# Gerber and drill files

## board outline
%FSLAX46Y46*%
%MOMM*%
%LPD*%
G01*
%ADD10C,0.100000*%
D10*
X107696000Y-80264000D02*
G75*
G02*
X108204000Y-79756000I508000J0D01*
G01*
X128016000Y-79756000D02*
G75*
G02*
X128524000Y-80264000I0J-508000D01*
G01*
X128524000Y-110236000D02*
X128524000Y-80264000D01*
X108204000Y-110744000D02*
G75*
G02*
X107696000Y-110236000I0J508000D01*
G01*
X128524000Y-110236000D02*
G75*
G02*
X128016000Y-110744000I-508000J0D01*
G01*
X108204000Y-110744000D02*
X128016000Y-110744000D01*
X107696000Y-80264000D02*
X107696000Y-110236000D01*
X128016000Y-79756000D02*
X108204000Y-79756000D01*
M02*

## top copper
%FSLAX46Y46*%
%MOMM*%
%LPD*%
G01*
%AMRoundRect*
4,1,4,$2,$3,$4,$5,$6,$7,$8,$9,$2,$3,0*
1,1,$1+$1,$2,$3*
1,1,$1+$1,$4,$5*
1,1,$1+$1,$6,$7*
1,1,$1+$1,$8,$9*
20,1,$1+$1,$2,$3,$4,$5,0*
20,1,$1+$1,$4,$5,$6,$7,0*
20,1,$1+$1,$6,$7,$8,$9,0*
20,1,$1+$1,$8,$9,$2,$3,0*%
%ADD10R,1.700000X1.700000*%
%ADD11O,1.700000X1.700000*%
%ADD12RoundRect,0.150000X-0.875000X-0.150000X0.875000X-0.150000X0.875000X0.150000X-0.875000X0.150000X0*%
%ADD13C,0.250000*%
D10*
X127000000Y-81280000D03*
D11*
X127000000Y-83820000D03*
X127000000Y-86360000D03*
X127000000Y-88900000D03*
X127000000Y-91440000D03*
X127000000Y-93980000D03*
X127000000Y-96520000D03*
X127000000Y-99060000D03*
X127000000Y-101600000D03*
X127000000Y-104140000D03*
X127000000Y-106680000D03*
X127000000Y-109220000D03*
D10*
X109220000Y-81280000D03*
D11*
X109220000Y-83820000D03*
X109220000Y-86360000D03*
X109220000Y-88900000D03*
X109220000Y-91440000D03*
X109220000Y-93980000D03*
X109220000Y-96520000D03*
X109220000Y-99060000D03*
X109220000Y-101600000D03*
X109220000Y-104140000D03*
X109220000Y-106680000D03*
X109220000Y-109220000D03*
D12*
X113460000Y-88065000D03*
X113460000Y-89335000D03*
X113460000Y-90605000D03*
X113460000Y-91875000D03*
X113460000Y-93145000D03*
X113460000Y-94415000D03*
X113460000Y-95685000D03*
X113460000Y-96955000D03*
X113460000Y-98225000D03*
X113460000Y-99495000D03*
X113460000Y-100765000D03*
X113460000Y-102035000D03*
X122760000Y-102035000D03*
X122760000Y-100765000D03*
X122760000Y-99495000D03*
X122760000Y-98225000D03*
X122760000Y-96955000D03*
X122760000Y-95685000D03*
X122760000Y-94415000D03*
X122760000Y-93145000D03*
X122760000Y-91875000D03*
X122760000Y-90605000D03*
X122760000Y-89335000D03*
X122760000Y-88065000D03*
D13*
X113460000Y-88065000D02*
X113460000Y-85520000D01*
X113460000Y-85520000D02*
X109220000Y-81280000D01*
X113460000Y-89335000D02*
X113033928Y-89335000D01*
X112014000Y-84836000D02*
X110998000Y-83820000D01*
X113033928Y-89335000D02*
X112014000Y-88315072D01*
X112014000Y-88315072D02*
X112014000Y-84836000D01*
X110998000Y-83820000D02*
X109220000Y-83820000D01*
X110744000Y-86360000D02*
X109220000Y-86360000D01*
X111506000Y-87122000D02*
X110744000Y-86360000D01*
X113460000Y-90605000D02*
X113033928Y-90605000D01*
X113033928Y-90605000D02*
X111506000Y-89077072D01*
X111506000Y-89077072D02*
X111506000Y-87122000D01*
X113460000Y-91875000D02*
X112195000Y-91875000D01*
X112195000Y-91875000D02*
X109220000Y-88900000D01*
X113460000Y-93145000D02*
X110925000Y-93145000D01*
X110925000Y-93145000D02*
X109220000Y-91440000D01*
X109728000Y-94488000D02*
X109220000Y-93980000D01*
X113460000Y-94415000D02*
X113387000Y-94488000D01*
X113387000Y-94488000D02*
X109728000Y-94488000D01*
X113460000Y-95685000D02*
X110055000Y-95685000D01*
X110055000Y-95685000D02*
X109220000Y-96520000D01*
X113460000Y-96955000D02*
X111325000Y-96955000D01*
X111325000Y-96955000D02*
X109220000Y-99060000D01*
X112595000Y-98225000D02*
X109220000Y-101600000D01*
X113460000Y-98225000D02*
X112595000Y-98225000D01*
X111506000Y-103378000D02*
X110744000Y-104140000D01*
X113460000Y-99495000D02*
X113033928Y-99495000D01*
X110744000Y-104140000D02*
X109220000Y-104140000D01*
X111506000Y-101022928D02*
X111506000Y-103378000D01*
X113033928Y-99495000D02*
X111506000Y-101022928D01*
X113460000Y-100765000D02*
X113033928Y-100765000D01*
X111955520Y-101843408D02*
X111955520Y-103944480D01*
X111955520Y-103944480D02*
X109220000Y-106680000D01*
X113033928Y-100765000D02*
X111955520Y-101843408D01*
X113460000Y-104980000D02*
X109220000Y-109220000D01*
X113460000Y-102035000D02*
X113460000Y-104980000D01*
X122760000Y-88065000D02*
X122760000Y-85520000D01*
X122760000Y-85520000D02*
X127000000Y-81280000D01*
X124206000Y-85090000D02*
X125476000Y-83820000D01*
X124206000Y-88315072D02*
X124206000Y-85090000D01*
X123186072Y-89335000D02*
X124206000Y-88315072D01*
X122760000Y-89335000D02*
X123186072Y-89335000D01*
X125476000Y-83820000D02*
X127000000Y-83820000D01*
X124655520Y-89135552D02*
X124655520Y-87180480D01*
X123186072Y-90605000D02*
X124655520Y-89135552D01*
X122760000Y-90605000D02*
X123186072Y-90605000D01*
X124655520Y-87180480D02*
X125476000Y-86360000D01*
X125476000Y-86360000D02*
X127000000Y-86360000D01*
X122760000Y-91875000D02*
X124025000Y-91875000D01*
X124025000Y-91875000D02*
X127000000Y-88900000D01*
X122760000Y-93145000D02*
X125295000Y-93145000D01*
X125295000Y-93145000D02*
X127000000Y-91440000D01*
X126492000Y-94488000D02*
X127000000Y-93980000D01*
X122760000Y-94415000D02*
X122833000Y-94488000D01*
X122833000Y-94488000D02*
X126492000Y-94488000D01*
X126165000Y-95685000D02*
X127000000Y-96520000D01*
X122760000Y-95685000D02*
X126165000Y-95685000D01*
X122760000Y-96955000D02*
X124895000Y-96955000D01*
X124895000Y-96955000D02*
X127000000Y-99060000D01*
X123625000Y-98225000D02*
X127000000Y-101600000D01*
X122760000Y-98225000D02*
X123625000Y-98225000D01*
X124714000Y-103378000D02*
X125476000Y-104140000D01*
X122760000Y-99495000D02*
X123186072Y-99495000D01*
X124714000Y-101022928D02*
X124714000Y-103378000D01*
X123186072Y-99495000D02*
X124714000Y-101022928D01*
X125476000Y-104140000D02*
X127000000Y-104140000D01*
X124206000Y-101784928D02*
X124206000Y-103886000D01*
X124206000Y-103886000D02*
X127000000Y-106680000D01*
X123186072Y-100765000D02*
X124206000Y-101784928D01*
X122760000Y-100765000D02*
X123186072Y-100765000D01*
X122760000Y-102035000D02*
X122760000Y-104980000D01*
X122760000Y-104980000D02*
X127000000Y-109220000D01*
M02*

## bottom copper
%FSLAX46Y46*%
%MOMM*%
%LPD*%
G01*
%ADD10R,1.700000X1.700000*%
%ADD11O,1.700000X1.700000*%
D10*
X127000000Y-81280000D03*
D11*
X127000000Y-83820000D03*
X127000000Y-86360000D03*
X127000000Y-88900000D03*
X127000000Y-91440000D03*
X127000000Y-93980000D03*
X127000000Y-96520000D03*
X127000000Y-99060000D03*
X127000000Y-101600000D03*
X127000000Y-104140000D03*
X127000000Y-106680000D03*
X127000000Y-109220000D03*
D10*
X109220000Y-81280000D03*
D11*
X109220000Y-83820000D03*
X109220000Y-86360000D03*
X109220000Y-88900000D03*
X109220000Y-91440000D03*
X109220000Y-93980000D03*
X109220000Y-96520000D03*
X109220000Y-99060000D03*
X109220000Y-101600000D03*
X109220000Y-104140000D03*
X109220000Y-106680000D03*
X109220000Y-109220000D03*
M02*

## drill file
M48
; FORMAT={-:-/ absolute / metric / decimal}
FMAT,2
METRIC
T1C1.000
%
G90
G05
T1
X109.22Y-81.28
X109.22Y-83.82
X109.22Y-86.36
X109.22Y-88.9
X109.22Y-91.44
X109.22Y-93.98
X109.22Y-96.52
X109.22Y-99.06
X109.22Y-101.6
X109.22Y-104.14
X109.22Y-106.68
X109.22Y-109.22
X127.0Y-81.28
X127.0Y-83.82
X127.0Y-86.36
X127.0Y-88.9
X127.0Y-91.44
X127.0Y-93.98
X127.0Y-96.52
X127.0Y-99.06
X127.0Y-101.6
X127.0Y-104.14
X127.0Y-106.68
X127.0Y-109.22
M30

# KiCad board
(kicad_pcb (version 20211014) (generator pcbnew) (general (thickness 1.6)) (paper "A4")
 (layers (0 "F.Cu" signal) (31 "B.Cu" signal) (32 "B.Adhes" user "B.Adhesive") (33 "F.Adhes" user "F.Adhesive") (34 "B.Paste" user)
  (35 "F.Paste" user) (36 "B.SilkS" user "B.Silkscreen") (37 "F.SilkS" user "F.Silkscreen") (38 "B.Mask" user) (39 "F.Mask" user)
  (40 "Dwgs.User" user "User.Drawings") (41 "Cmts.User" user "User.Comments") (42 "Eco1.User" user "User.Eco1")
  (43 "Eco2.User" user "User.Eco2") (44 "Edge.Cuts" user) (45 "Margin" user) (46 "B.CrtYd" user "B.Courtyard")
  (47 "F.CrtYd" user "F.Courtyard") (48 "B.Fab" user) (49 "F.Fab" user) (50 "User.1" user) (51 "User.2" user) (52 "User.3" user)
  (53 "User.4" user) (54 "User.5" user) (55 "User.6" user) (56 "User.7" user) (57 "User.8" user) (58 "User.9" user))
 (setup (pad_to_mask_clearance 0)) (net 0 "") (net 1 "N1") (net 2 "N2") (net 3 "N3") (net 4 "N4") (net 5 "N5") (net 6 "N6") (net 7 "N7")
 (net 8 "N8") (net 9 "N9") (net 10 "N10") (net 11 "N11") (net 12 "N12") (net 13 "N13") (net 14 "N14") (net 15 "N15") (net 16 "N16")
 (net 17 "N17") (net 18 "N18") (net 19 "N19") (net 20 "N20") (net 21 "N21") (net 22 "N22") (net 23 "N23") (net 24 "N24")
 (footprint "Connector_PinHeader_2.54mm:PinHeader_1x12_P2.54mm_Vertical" (layer "F.Cu") (at 127 81.28)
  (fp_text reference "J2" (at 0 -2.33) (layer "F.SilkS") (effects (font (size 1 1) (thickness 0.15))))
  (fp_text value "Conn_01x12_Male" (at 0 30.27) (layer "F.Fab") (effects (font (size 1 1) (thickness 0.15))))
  (pad "1" thru_hole rect locked (at 0 0) (size 1.7 1.7) (drill 1) (layers *.Cu *.Mask) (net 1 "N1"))
  (pad "2" thru_hole oval locked (at 0 2.54) (size 1.7 1.7) (drill 1) (layers *.Cu *.Mask) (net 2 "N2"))
  (pad "3" thru_hole oval locked (at 0 5.08) (size 1.7 1.7) (drill 1) (layers *.Cu *.Mask) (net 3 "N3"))
  (pad "4" thru_hole oval locked (at 0 7.62) (size 1.7 1.7) (drill 1) (layers *.Cu *.Mask) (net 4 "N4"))
  (pad "5" thru_hole oval locked (at 0 10.16) (size 1.7 1.7) (drill 1) (layers *.Cu *.Mask) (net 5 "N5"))
  (pad "6" thru_hole oval locked (at 0 12.7) (size 1.7 1.7) (drill 1) (layers *.Cu *.Mask) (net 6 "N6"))
  (pad "7" thru_hole oval locked (at 0 15.24) (size 1.7 1.7) (drill 1) (layers *.Cu *.Mask) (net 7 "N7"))
  (pad "8" thru_hole oval locked (at 0 17.78) (size 1.7 1.7) (drill 1) (layers *.Cu *.Mask) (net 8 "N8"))
  (pad "9" thru_hole oval locked (at 0 20.32) (size 1.7 1.7) (drill 1) (layers *.Cu *.Mask) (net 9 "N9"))
  (pad "10" thru_hole oval locked (at 0 22.86) (size 1.7 1.7) (drill 1) (layers *.Cu *.Mask) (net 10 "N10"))
  (pad "11" thru_hole oval locked (at 0 25.4) (size 1.7 1.7) (drill 1) (layers *.Cu *.Mask) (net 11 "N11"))
  (pad "12" thru_hole oval locked (at 0 27.94) (size 1.7 1.7) (drill 1) (layers *.Cu *.Mask) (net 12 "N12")))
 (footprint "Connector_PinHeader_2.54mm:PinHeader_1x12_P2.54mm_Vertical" (layer "F.Cu") (at 109.22 81.28)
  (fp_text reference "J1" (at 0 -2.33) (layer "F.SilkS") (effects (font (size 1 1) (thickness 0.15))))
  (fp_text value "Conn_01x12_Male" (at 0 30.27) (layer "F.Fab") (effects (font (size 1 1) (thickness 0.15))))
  (pad "1" thru_hole rect locked (at 0 0) (size 1.7 1.7) (drill 1) (layers *.Cu *.Mask) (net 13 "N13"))
  (pad "2" thru_hole oval locked (at 0 2.54) (size 1.7 1.7) (drill 1) (layers *.Cu *.Mask) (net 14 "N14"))
  (pad "3" thru_hole oval locked (at 0 5.08) (size 1.7 1.7) (drill 1) (layers *.Cu *.Mask) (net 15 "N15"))
  (pad "4" thru_hole oval locked (at 0 7.62) (size 1.7 1.7) (drill 1) (layers *.Cu *.Mask) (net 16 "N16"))
  (pad "5" thru_hole oval locked (at 0 10.16) (size 1.7 1.7) (drill 1) (layers *.Cu *.Mask) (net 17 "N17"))
  (pad "6" thru_hole oval locked (at 0 12.7) (size 1.7 1.7) (drill 1) (layers *.Cu *.Mask) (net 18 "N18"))
  (pad "7" thru_hole oval locked (at 0 15.24) (size 1.7 1.7) (drill 1) (layers *.Cu *.Mask) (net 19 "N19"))
  (pad "8" thru_hole oval locked (at 0 17.78) (size 1.7 1.7) (drill 1) (layers *.Cu *.Mask) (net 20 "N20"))
  (pad "9" thru_hole oval locked (at 0 20.32) (size 1.7 1.7) (drill 1) (layers *.Cu *.Mask) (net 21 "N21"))
  (pad "10" thru_hole oval locked (at 0 22.86) (size 1.7 1.7) (drill 1) (layers *.Cu *.Mask) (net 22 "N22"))
  (pad "11" thru_hole oval locked (at 0 25.4) (size 1.7 1.7) (drill 1) (layers *.Cu *.Mask) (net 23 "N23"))
  (pad "12" thru_hole oval locked (at 0 27.94) (size 1.7 1.7) (drill 1) (layers *.Cu *.Mask) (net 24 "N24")))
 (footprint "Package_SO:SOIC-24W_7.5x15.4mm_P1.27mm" (layer "F.Cu") (at 118.11 95.05)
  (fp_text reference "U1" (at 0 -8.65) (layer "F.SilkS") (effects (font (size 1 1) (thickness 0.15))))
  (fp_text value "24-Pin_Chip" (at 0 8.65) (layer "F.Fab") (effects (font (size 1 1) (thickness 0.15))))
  (pad "1" smd roundrect locked (at -4.65 -6.985) (size 2.05 0.6) (layers "F.Cu" "F.Paste" "F.Mask") (roundrect_rratio 0.25) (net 13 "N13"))
  (pad "2" smd roundrect locked (at -4.65 -5.715) (size 2.05 0.6) (layers "F.Cu" "F.Paste" "F.Mask") (roundrect_rratio 0.25) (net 14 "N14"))
  (pad "3" smd roundrect locked (at -4.65 -4.445) (size 2.05 0.6) (layers "F.Cu" "F.Paste" "F.Mask") (roundrect_rratio 0.25) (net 15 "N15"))
  (pad "4" smd roundrect locked (at -4.65 -3.175) (size 2.05 0.6) (layers "F.Cu" "F.Paste" "F.Mask") (roundrect_rratio 0.25) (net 16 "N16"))
  (pad "5" smd roundrect locked (at -4.65 -1.905) (size 2.05 0.6) (layers "F.Cu" "F.Paste" "F.Mask") (roundrect_rratio 0.25) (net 17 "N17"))
  (pad "6" smd roundrect locked (at -4.65 -0.635) (size 2.05 0.6) (layers "F.Cu" "F.Paste" "F.Mask") (roundrect_rratio 0.25) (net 18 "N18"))
  (pad "7" smd roundrect locked (at -4.65 0.635) (size 2.05 0.6) (layers "F.Cu" "F.Paste" "F.Mask") (roundrect_rratio 0.25) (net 19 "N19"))
  (pad "8" smd roundrect locked (at -4.65 1.905) (size 2.05 0.6) (layers "F.Cu" "F.Paste" "F.Mask") (roundrect_rratio 0.25) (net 20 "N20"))
  (pad "9" smd roundrect locked (at -4.65 3.175) (size 2.05 0.6) (layers "F.Cu" "F.Paste" "F.Mask") (roundrect_rratio 0.25) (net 21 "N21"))
  (pad "10" smd roundrect locked (at -4.65 4.445) (size 2.05 0.6) (layers "F.Cu" "F.Paste" "F.Mask") (roundrect_rratio 0.25) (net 22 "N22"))
  (pad "11" smd roundrect locked (at -4.65 5.715) (size 2.05 0.6) (layers "F.Cu" "F.Paste" "F.Mask") (roundrect_rratio 0.25) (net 23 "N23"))
  (pad "12" smd roundrect locked (at -4.65 6.985) (size 2.05 0.6) (layers "F.Cu" "F.Paste" "F.Mask") (roundrect_rratio 0.25) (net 24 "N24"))
  (pad "13" smd roundrect locked (at 4.65 6.985) (size 2.05 0.6) (layers "F.Cu" "F.Paste" "F.Mask") (roundrect_rratio 0.25) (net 12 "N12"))
  (pad "14" smd roundrect locked (at 4.65 5.715) (size 2.05 0.6) (layers "F.Cu" "F.Paste" "F.Mask") (roundrect_rratio 0.25) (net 11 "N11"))
  (pad "15" smd roundrect locked (at 4.65 4.445) (size 2.05 0.6) (layers "F.Cu" "F.Paste" "F.Mask") (roundrect_rratio 0.25) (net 10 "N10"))
  (pad "16" smd roundrect locked (at 4.65 3.175) (size 2.05 0.6) (layers "F.Cu" "F.Paste" "F.Mask") (roundrect_rratio 0.25) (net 9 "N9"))
  (pad "17" smd roundrect locked (at 4.65 1.905) (size 2.05 0.6) (layers "F.Cu" "F.Paste" "F.Mask") (roundrect_rratio 0.25) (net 8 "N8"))
  (pad "18" smd roundrect locked (at 4.65 0.635) (size 2.05 0.6) (layers "F.Cu" "F.Paste" "F.Mask") (roundrect_rratio 0.25) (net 7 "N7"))
  (pad "19" smd roundrect locked (at 4.65 -0.635) (size 2.05 0.6) (layers "F.Cu" "F.Paste" "F.Mask") (roundrect_rratio 0.25) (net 6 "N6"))
  (pad "20" smd roundrect locked (at 4.65 -1.905) (size 2.05 0.6) (layers "F.Cu" "F.Paste" "F.Mask") (roundrect_rratio 0.25) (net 5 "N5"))
  (pad "21" smd roundrect locked (at 4.65 -3.175) (size 2.05 0.6) (layers "F.Cu" "F.Paste" "F.Mask") (roundrect_rratio 0.25) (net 4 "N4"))
  (pad "22" smd roundrect locked (at 4.65 -4.445) (size 2.05 0.6) (layers "F.Cu" "F.Paste" "F.Mask") (roundrect_rratio 0.25) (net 3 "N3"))
  (pad "23" smd roundrect locked (at 4.65 -5.715) (size 2.05 0.6) (layers "F.Cu" "F.Paste" "F.Mask") (roundrect_rratio 0.25) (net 2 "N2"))
  (pad "24" smd roundrect locked (at 4.65 -6.985) (size 2.05 0.6) (layers "F.Cu" "F.Paste" "F.Mask") (roundrect_rratio 0.25) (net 1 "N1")))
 (gr_arc (start 107.696 80.264) (mid 107.84479 79.90479) (end 108.204 79.756) (layer "Edge.Cuts") (width 0.1))
 (gr_arc (start 128.016 79.756) (mid 128.37521 79.90479) (end 128.524 80.264) (layer "Edge.Cuts") (width 0.1))
 (gr_line (start 128.524 110.236) (end 128.524 80.264) (layer "Edge.Cuts") (width 0.1))
 (gr_arc (start 108.204 110.744) (mid 107.84479 110.59521) (end 107.696 110.236) (layer "Edge.Cuts") (width 0.1))
 (gr_arc (start 128.524 110.236) (mid 128.37521 110.59521) (end 128.016 110.744) (layer "Edge.Cuts") (width 0.1))
 (gr_line (start 108.204 110.744) (end 128.016 110.744) (layer "Edge.Cuts") (width 0.1))
 (gr_line (start 107.696 80.264) (end 107.696 110.236) (layer "Edge.Cuts") (width 0.1))
 (gr_line (start 128.016 79.756) (end 108.204 79.756) (layer "Edge.Cuts") (width 0.1))
 (segment (start 113.46 88.065) (end 113.46 85.52) (width 0.25) (layer "F.Cu") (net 13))
 (segment (start 113.46 85.52) (end 109.22 81.28) (width 0.25) (layer "F.Cu") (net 13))
 (segment (start 113.46 89.335) (end 113.033928 89.335) (width 0.25) (layer "F.Cu") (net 14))
 (segment (start 112.014 84.836) (end 110.998 83.82) (width 0.25) (layer "F.Cu") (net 14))
 (segment (start 113.033928 89.335) (end 112.014 88.315072) (width 0.25) (layer "F.Cu") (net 14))
 (segment (start 112.014 88.315072) (end 112.014 84.836) (width 0.25) (layer "F.Cu") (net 14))
 (segment (start 110.998 83.82) (end 109.22 83.82) (width 0.25) (layer "F.Cu") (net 14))
 (segment (start 110.744 86.36) (end 109.22 86.36) (width 0.25) (layer "F.Cu") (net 15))
 (segment (start 111.506 87.122) (end 110.744 86.36) (width 0.25) (layer "F.Cu") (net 15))
 (segment (start 113.46 90.605) (end 113.033928 90.605) (width 0.25) (layer "F.Cu") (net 15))
 (segment (start 113.033928 90.605) (end 111.506 89.077072) (width 0.25) (layer "F.Cu") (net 15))
 (segment (start 111.506 89.077072) (end 111.506 87.122) (width 0.25) (layer "F.Cu") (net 15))
 (segment (start 113.46 91.875) (end 112.195 91.875) (width 0.25) (layer "F.Cu") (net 16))
 (segment (start 112.195 91.875) (end 109.22 88.9) (width 0.25) (layer "F.Cu") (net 16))
 (segment (start 113.46 93.145) (end 110.925 93.145) (width 0.25) (layer "F.Cu") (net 17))
 (segment (start 110.925 93.145) (end 109.22 91.44) (width 0.25) (layer "F.Cu") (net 17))
 (segment (start 109.728 94.488) (end 109.22 93.98) (width 0.25) (layer "F.Cu") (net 18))
 (segment (start 113.46 94.415) (end 113.387 94.488) (width 0.25) (layer "F.Cu") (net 18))
 (segment (start 113.387 94.488) (end 109.728 94.488) (width 0.25) (layer "F.Cu") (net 18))
 (segment (start 113.46 95.685) (end 110.055 95.685) (width 0.25) (layer "F.Cu") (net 19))
 (segment (start 110.055 95.685) (end 109.22 96.52) (width 0.25) (layer "F.Cu") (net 19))
 (segment (start 113.46 96.955) (end 111.325 96.955) (width 0.25) (layer "F.Cu") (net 20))
 (segment (start 111.325 96.955) (end 109.22 99.06) (width 0.25) (layer "F.Cu") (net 20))
 (segment (start 112.595 98.225) (end 109.22 101.6) (width 0.25) (layer "F.Cu") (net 21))
 (segment (start 113.46 98.225) (end 112.595 98.225) (width 0.25) (layer "F.Cu") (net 21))
 (segment (start 111.506 103.378) (end 110.744 104.14) (width 0.25) (layer "F.Cu") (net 22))
 (segment (start 113.46 99.495) (end 113.033928 99.495) (width 0.25) (layer "F.Cu") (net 22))
 (segment (start 110.744 104.14) (end 109.22 104.14) (width 0.25) (layer "F.Cu") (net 22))
 (segment (start 111.506 101.022928) (end 111.506 103.378) (width 0.25) (layer "F.Cu") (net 22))
 (segment (start 113.033928 99.495) (end 111.506 101.022928) (width 0.25) (layer "F.Cu") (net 22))
 (segment (start 113.46 100.765) (end 113.033928 100.765) (width 0.25) (layer "F.Cu") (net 23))
 (segment (start 111.95552 101.843408) (end 111.95552 103.94448) (width 0.25) (layer "F.Cu") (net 23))
 (segment (start 111.95552 103.94448) (end 109.22 106.68) (width 0.25) (layer "F.Cu") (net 23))
 (segment (start 113.033928 100.765) (end 111.95552 101.843408) (width 0.25) (layer "F.Cu") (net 23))
 (segment (start 113.46 104.98) (end 109.22 109.22) (width 0.25) (layer "F.Cu") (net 24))
 (segment (start 113.46 102.035) (end 113.46 104.98) (width 0.25) (layer "F.Cu") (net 24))
 (segment (start 122.76 88.065) (end 122.76 85.52) (width 0.25) (layer "F.Cu") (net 1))
 (segment (start 122.76 85.52) (end 127 81.28) (width 0.25) (layer "F.Cu") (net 1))
 (segment (start 124.206 85.09) (end 125.476 83.82) (width 0.25) (layer "F.Cu") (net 2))
 (segment (start 124.206 88.315072) (end 124.206 85.09) (width 0.25) (layer "F.Cu") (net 2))
 (segment (start 123.186072 89.335) (end 124.206 88.315072) (width 0.25) (layer "F.Cu") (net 2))
 (segment (start 122.76 89.335) (end 123.186072 89.335) (width 0.25) (layer "F.Cu") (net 2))
 (segment (start 125.476 83.82) (end 127 83.82) (width 0.25) (layer "F.Cu") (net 2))
 (segment (start 124.65552 89.135552) (end 124.65552 87.18048) (width 0.25) (layer "F.Cu") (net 3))
 (segment (start 123.186072 90.605) (end 124.65552 89.135552) (width 0.25) (layer "F.Cu") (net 3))
 (segment (start 122.76 90.605) (end 123.186072 90.605) (width 0.25) (layer "F.Cu") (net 3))
 (segment (start 124.65552 87.18048) (end 125.476 86.36) (width 0.25) (layer "F.Cu") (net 3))
 (segment (start 125.476 86.36) (end 127 86.36) (width 0.25) (layer "F.Cu") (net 3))
 (segment (start 122.76 91.875) (end 124.025 91.875) (width 0.25) (layer "F.Cu") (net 4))
 (segment (start 124.025 91.875) (end 127 88.9) (width 0.25) (layer "F.Cu") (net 4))
 (segment (start 122.76 93.145) (end 125.295 93.145) (width 0.25) (layer "F.Cu") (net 5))
 (segment (start 125.295 93.145) (end 127 91.44) (width 0.25) (layer "F.Cu") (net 5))
 (segment (start 126.492 94.488) (end 127 93.98) (width 0.25) (layer "F.Cu") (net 6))
 (segment (start 122.76 94.415) (end 122.833 94.488) (width 0.25) (layer "F.Cu") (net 6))
 (segment (start 122.833 94.488) (end 126.492 94.488) (width 0.25) (layer "F.Cu") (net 6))
 (segment (start 126.165 95.685) (end 127 96.52) (width 0.25) (layer "F.Cu") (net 7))
 (segment (start 122.76 95.685) (end 126.165 95.685) (width 0.25) (layer "F.Cu") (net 7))
 (segment (start 122.76 96.955) (end 124.895 96.955) (width 0.25) (layer "F.Cu") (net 8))
 (segment (start 124.895 96.955) (end 127 99.06) (width 0.25) (layer "F.Cu") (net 8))
 (segment (start 123.625 98.225) (end 127 101.6) (width 0.25) (layer "F.Cu") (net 9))
 (segment (start 122.76 98.225) (end 123.625 98.225) (width 0.25) (layer "F.Cu") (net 9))
 (segment (start 124.714 103.378) (end 125.476 104.14) (width 0.25) (layer "F.Cu") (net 10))
 (segment (start 122.76 99.495) (end 123.186072 99.495) (width 0.25) (layer "F.Cu") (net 10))
 (segment (start 124.714 101.022928) (end 124.714 103.378) (width 0.25) (layer "F.Cu") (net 10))
 (segment (start 123.186072 99.495) (end 124.714 101.022928) (width 0.25) (layer "F.Cu") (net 10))
 (segment (start 125.476 104.14) (end 127 104.14) (width 0.25) (layer "F.Cu") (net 10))
 (segment (start 124.206 101.784928) (end 124.206 103.886) (width 0.25) (layer "F.Cu") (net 11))
 (segment (start 124.206 103.886) (end 127 106.68) (width 0.25) (layer "F.Cu") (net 11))
 (segment (start 123.186072 100.765) (end 124.206 101.784928) (width 0.25) (layer "F.Cu") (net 11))
 (segment (start 122.76 100.765) (end 123.186072 100.765) (width 0.25) (layer "F.Cu") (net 11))
 (segment (start 122.76 102.035) (end 122.76 104.98) (width 0.25) (layer "F.Cu") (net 12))
 (segment (start 122.76 104.98) (end 127 109.22) (width 0.25) (layer "F.Cu") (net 12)))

